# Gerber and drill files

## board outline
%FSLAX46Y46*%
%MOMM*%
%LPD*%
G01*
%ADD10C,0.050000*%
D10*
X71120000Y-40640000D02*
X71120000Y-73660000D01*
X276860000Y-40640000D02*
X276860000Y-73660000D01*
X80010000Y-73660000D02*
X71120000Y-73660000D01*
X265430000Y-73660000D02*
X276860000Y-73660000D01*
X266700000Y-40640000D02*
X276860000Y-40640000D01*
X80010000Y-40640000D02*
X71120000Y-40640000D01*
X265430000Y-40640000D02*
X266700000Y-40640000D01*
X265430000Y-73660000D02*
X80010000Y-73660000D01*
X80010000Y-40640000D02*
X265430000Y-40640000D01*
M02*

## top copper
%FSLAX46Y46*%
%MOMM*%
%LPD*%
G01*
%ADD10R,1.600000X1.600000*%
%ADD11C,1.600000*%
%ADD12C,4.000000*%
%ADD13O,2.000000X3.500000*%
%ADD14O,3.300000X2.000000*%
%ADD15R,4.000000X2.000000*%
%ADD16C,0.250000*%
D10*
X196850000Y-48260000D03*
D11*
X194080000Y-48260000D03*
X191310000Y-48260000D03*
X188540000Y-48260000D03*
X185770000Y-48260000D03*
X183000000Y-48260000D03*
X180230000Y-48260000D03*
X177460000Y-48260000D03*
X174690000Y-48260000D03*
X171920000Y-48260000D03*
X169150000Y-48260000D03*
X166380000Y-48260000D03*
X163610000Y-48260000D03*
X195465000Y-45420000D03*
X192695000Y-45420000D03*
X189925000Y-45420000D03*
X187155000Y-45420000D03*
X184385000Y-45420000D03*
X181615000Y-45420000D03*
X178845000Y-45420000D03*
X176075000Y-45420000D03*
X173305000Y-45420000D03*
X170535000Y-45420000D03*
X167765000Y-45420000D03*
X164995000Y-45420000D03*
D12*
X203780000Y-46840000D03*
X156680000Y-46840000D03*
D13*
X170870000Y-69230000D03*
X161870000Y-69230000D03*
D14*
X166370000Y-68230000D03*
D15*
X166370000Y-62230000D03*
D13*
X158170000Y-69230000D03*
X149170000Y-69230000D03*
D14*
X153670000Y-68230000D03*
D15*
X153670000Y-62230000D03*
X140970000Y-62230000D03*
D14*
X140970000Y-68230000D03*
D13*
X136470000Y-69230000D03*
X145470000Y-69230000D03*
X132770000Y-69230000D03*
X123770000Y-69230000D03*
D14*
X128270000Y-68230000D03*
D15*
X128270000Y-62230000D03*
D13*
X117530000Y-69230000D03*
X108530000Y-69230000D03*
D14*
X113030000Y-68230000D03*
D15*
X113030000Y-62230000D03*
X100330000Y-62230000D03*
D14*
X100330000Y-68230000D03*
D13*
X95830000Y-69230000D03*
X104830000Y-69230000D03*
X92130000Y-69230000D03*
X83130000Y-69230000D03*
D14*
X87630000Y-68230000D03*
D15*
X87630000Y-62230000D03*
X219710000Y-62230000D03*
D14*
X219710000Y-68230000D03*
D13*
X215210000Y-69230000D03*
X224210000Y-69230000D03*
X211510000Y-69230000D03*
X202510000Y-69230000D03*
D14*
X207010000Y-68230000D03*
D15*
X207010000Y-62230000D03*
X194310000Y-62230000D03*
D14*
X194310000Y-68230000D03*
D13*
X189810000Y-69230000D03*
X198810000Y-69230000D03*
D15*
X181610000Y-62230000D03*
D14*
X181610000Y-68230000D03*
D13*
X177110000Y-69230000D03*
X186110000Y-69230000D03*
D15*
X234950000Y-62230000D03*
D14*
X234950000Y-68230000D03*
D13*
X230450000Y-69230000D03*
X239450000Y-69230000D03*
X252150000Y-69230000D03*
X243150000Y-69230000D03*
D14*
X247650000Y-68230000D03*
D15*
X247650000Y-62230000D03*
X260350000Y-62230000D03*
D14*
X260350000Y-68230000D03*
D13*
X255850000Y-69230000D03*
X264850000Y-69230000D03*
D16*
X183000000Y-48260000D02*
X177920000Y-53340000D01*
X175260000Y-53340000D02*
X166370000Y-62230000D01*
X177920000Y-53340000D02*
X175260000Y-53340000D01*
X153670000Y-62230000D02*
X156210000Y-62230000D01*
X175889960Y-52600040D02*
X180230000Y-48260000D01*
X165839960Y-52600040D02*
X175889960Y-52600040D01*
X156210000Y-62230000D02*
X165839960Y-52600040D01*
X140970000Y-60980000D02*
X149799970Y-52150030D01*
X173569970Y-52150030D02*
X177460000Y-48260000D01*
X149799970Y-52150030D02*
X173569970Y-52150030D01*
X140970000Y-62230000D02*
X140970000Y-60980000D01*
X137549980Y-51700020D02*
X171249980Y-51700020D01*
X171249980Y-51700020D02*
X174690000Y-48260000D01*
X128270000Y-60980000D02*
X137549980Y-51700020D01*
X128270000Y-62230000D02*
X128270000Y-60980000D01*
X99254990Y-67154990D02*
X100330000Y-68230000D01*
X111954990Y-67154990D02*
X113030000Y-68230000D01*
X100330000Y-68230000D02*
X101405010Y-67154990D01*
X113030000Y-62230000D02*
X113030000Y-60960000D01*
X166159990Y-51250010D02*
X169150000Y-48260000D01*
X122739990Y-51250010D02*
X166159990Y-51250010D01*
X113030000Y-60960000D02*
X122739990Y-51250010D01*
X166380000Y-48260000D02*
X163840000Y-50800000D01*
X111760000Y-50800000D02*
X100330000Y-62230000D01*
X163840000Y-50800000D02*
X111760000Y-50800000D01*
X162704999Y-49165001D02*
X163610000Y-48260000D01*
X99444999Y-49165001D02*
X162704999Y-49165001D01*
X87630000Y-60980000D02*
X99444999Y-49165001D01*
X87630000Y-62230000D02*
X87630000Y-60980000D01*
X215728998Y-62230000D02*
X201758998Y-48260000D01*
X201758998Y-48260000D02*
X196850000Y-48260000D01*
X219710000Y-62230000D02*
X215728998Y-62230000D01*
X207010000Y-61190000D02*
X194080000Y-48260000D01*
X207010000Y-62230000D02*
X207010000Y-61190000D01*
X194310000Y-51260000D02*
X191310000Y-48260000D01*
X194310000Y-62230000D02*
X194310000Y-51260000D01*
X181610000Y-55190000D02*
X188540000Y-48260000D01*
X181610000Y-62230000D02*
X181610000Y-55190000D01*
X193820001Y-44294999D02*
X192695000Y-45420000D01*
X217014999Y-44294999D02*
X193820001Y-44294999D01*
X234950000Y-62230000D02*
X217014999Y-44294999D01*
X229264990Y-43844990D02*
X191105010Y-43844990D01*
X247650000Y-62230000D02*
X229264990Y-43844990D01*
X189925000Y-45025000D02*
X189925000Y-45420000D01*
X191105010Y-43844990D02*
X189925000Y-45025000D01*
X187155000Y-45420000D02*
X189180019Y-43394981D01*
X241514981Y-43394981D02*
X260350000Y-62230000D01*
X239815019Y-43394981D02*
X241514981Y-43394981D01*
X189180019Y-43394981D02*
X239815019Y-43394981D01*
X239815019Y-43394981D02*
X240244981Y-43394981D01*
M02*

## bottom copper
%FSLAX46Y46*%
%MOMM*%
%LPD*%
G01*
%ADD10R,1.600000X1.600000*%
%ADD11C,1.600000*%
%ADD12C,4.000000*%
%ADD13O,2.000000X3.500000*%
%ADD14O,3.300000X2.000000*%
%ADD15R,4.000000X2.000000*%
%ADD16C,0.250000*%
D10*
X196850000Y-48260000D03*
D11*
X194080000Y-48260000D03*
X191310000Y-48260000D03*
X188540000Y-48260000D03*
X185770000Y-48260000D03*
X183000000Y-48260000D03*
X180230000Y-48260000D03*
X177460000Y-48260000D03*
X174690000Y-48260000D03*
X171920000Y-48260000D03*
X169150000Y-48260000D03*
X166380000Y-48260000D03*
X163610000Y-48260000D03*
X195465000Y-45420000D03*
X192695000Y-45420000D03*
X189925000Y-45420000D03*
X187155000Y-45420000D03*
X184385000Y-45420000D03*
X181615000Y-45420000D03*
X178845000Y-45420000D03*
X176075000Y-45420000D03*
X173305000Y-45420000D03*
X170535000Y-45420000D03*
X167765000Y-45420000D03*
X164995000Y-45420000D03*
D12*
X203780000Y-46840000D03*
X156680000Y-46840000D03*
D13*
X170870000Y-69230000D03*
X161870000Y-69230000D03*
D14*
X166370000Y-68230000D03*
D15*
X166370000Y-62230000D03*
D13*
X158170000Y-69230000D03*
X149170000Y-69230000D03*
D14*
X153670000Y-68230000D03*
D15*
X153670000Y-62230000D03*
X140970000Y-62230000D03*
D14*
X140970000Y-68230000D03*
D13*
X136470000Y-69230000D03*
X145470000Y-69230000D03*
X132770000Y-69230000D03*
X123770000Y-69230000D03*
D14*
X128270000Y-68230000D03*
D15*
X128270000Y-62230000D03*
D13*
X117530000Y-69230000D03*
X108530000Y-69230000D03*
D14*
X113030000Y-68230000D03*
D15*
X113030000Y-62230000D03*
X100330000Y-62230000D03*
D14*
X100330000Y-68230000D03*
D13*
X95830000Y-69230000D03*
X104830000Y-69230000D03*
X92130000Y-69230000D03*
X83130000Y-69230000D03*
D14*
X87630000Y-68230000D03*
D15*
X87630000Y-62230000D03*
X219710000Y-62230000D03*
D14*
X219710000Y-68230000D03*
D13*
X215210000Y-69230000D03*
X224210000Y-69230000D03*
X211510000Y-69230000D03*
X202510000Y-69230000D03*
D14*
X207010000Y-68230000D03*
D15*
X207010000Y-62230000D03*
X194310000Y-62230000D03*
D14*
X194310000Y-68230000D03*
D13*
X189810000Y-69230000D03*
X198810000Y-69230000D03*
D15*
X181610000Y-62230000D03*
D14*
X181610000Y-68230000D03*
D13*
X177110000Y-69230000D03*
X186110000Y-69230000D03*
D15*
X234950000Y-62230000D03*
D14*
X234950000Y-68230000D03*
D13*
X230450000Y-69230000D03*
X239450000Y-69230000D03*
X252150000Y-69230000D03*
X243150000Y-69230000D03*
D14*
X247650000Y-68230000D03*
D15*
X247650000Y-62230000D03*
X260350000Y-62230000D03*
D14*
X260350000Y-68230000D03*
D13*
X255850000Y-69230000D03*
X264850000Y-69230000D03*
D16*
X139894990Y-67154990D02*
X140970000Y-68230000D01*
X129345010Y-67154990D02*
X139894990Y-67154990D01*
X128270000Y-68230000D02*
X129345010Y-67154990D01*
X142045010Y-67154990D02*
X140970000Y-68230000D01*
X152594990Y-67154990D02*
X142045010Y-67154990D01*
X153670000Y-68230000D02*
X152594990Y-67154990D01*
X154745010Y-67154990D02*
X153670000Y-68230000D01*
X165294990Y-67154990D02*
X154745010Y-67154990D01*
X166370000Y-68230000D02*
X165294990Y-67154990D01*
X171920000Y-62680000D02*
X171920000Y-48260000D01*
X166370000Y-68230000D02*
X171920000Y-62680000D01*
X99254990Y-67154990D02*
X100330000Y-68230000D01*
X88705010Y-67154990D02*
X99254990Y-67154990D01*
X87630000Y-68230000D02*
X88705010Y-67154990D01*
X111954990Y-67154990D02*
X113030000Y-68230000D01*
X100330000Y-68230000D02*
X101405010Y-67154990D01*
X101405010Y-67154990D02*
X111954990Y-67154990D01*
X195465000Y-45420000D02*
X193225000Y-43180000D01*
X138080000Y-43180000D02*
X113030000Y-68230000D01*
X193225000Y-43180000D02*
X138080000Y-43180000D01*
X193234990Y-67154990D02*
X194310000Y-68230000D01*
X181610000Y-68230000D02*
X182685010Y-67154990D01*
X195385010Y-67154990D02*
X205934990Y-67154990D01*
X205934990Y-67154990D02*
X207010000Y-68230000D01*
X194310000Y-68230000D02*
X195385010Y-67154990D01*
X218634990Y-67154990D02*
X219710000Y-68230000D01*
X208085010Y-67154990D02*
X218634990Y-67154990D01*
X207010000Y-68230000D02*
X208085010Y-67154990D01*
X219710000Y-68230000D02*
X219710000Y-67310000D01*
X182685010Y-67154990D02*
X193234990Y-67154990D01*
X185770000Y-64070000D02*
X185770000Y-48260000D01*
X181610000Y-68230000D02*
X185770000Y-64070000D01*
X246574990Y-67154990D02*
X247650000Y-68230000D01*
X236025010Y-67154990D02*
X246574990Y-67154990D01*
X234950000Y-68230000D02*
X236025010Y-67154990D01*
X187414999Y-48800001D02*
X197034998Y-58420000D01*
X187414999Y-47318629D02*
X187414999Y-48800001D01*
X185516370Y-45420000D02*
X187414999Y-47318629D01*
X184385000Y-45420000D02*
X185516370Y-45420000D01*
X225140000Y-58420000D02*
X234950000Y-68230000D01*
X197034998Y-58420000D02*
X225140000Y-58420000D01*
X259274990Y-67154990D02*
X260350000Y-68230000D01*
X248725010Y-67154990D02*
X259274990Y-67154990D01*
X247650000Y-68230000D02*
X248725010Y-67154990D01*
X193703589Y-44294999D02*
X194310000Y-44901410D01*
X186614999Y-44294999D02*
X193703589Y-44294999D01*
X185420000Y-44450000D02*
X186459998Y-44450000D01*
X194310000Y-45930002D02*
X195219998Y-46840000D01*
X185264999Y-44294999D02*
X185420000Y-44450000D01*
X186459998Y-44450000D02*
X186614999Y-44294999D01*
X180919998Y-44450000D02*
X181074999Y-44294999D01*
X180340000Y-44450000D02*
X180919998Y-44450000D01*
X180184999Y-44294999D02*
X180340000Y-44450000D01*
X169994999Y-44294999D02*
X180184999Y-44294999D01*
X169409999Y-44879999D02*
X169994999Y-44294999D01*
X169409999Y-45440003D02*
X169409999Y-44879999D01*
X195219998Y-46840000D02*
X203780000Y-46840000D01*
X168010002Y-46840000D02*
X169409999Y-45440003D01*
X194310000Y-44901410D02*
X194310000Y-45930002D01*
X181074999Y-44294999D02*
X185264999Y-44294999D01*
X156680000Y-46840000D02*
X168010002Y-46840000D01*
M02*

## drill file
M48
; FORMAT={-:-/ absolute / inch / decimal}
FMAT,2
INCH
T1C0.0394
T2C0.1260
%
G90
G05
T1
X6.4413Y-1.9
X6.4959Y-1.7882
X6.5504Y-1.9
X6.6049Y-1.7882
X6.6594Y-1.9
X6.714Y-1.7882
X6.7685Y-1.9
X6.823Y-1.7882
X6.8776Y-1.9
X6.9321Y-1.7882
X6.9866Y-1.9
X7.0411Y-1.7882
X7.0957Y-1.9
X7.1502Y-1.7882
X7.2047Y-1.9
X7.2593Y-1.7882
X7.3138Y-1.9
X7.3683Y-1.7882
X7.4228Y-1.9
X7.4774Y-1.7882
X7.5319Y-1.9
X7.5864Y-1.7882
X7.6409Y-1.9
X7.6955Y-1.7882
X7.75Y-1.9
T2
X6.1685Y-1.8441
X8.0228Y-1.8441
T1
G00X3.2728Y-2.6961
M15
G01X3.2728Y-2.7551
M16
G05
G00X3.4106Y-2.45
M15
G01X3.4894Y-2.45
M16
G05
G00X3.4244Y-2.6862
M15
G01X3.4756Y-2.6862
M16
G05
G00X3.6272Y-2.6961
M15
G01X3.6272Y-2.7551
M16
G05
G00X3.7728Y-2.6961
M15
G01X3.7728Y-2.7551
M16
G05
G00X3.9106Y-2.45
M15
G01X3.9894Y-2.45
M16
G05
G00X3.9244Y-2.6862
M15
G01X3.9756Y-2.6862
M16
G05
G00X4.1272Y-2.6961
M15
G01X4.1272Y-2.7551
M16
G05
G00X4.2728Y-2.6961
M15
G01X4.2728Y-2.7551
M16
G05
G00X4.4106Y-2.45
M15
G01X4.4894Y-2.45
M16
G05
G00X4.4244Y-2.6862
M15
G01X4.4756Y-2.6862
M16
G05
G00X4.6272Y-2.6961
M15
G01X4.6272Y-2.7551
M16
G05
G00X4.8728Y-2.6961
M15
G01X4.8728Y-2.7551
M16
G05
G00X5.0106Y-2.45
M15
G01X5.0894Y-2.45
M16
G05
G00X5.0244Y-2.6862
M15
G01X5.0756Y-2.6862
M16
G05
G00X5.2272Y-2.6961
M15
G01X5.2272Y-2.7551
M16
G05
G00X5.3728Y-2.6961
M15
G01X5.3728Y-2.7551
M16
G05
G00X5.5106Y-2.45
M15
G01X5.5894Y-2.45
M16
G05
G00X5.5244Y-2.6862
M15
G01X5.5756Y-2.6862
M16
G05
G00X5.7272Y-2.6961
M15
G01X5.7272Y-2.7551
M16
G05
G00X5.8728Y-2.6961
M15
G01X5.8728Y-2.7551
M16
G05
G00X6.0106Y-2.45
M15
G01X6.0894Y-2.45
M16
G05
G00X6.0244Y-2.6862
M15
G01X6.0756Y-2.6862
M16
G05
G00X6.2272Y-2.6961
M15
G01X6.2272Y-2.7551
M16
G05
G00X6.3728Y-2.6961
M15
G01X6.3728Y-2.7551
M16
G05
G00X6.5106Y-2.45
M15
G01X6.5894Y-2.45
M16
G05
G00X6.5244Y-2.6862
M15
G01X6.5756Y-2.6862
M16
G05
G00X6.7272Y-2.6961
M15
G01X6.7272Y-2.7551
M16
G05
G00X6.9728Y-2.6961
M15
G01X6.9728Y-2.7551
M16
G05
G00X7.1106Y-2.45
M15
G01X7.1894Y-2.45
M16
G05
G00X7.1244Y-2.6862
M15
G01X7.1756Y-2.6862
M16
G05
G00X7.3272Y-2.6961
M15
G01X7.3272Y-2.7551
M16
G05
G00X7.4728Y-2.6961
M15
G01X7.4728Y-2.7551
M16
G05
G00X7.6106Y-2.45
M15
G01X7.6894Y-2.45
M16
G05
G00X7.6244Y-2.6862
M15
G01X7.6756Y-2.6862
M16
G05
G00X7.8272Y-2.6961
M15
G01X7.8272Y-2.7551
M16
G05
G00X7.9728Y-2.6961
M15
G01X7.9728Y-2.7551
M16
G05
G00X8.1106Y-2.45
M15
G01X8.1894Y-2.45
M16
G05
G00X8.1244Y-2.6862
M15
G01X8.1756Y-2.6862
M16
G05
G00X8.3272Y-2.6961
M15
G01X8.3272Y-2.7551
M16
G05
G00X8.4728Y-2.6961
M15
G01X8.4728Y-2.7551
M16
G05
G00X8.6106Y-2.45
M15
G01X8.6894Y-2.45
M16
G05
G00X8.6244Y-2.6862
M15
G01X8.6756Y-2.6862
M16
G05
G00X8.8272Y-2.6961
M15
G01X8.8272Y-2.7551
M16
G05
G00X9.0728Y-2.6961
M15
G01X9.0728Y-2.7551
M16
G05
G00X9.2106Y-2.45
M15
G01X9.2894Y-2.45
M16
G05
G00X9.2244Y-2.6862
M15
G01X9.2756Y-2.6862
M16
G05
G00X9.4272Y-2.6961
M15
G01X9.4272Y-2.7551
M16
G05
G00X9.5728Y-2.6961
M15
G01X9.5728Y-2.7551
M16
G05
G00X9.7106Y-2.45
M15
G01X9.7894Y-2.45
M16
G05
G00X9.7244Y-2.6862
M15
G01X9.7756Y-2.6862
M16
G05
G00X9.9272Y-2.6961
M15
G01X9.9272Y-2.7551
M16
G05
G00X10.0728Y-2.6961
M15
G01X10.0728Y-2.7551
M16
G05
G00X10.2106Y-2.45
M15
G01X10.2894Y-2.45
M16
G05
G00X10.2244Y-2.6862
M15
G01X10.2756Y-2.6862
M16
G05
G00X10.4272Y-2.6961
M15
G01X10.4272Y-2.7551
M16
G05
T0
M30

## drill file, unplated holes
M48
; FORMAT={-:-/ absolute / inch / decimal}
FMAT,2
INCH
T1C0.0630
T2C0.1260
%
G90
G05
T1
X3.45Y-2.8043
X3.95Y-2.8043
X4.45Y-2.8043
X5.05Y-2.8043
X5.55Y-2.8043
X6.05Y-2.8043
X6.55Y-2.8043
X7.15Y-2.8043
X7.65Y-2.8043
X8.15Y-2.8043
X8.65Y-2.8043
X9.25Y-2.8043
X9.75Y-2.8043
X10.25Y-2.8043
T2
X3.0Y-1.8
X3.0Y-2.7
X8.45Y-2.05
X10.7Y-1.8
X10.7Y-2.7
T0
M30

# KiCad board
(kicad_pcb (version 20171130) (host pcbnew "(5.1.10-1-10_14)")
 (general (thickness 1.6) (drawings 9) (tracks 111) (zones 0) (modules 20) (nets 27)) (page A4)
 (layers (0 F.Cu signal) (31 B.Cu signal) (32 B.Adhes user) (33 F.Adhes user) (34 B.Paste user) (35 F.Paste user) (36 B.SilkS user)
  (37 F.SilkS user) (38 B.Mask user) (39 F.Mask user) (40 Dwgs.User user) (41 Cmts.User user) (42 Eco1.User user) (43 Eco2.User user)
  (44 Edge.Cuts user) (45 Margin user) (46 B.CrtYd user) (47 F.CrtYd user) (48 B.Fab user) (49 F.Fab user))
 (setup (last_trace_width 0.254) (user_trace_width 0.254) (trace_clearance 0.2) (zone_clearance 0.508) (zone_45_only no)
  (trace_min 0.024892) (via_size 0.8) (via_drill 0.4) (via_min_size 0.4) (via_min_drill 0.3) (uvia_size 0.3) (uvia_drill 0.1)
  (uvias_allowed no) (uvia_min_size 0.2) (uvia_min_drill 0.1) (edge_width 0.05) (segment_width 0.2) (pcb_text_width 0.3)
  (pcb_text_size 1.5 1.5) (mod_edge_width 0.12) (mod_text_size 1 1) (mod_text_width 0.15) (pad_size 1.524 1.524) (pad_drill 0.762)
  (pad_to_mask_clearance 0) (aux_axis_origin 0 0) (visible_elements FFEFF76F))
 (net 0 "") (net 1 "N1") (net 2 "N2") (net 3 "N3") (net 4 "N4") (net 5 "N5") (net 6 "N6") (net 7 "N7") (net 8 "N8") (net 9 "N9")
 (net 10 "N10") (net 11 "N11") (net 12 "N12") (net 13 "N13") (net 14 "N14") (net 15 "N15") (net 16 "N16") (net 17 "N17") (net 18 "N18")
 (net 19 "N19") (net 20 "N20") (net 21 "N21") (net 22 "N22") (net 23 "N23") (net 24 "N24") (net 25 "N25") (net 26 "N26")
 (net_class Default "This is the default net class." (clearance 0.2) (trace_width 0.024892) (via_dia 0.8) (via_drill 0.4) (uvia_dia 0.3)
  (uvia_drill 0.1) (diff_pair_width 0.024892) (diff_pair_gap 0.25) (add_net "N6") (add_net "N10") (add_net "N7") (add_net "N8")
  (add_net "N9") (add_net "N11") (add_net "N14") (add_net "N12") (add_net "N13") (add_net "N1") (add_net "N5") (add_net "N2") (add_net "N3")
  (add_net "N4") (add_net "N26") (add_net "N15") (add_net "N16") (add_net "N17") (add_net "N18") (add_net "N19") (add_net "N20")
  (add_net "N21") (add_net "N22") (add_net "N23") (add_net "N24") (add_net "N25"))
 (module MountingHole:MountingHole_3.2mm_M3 (layer F.Cu) (at 271.78 45.72)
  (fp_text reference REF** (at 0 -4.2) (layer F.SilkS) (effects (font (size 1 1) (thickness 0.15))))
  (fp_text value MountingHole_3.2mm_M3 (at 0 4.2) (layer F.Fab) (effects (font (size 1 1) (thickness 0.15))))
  (pad 1 np_thru_hole circle (at 0 0) (size 3.2 3.2) (drill 3.2) (layers *.Cu *.Mask)))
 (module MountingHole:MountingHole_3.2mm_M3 (layer F.Cu) (at 271.78 68.58)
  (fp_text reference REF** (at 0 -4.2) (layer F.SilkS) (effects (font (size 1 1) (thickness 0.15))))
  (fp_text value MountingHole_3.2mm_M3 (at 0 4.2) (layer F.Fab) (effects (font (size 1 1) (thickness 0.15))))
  (pad 1 np_thru_hole circle (at 0 0) (size 3.2 3.2) (drill 3.2) (layers *.Cu *.Mask)))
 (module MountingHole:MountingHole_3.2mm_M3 (layer F.Cu) (at 76.2 45.72)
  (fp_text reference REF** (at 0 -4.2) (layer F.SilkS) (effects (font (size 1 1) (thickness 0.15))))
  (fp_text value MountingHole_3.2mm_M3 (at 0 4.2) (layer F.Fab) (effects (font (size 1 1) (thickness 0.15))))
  (pad 1 np_thru_hole circle (at 0 0) (size 3.2 3.2) (drill 3.2) (layers *.Cu *.Mask)))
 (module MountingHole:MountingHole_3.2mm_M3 (layer F.Cu) (at 214.63 52.07)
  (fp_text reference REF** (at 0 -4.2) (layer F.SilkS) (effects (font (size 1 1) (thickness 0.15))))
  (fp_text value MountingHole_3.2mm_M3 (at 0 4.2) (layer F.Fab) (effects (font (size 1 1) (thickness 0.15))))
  (pad 1 np_thru_hole circle (at 0 0) (size 3.2 3.2) (drill 3.2) (layers *.Cu *.Mask)))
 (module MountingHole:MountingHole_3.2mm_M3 (layer F.Cu) (at 76.2 68.58)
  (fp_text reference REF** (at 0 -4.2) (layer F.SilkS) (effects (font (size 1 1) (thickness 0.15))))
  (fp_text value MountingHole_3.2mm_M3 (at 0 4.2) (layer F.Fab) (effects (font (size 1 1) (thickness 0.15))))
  (pad 1 np_thru_hole circle (at 0 0) (size 3.2 3.2) (drill 3.2) (layers *.Cu *.Mask)))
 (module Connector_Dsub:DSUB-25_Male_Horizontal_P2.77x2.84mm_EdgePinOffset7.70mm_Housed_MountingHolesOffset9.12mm (layer F.Cu)
  (at 196.85 48.26 180)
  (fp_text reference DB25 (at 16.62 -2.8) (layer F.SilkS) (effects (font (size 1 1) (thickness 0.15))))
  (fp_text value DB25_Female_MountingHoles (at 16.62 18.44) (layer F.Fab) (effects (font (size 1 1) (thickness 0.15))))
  (pad 1 thru_hole rect (at 0 0 180) (size 1.6 1.6) (drill 1) (layers *.Cu *.Mask) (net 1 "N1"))
  (pad 2 thru_hole circle (at 2.77 0 180) (size 1.6 1.6) (drill 1) (layers *.Cu *.Mask) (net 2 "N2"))
  (pad 3 thru_hole circle (at 5.54 0 180) (size 1.6 1.6) (drill 1) (layers *.Cu *.Mask) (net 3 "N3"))
  (pad 4 thru_hole circle (at 8.31 0 180) (size 1.6 1.6) (drill 1) (layers *.Cu *.Mask) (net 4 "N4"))
  (pad 5 thru_hole circle (at 11.08 0 180) (size 1.6 1.6) (drill 1) (layers *.Cu *.Mask) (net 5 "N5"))
  (pad 6 thru_hole circle (at 13.85 0 180) (size 1.6 1.6) (drill 1) (layers *.Cu *.Mask) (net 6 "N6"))
  (pad 7 thru_hole circle (at 16.62 0 180) (size 1.6 1.6) (drill 1) (layers *.Cu *.Mask) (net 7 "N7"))
  (pad 8 thru_hole circle (at 19.39 0 180) (size 1.6 1.6) (drill 1) (layers *.Cu *.Mask) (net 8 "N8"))
  (pad 9 thru_hole circle (at 22.16 0 180) (size 1.6 1.6) (drill 1) (layers *.Cu *.Mask) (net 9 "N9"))
  (pad 10 thru_hole circle (at 24.93 0 180) (size 1.6 1.6) (drill 1) (layers *.Cu *.Mask) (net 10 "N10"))
  (pad 11 thru_hole circle (at 27.7 0 180) (size 1.6 1.6) (drill 1) (layers *.Cu *.Mask) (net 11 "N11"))
  (pad 12 thru_hole circle (at 30.47 0 180) (size 1.6 1.6) (drill 1) (layers *.Cu *.Mask) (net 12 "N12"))
  (pad 13 thru_hole circle (at 33.24 0 180) (size 1.6 1.6) (drill 1) (layers *.Cu *.Mask) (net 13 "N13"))
  (pad 14 thru_hole circle (at 1.385 2.84 180) (size 1.6 1.6) (drill 1) (layers *.Cu *.Mask) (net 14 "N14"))
  (pad 15 thru_hole circle (at 4.155 2.84 180) (size 1.6 1.6) (drill 1) (layers *.Cu *.Mask) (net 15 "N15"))
  (pad 16 thru_hole circle (at 6.925 2.84 180) (size 1.6 1.6) (drill 1) (layers *.Cu *.Mask) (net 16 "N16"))
  (pad 17 thru_hole circle (at 9.695 2.84 180) (size 1.6 1.6) (drill 1) (layers *.Cu *.Mask) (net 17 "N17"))
  (pad 18 thru_hole circle (at 12.465 2.84 180) (size 1.6 1.6) (drill 1) (layers *.Cu *.Mask) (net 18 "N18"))
  (pad 19 thru_hole circle (at 15.235 2.84 180) (size 1.6 1.6) (drill 1) (layers *.Cu *.Mask) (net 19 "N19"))
  (pad 20 thru_hole circle (at 18.005 2.84 180) (size 1.6 1.6) (drill 1) (layers *.Cu *.Mask) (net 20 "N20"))
  (pad 21 thru_hole circle (at 20.775 2.84 180) (size 1.6 1.6) (drill 1) (layers *.Cu *.Mask) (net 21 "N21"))
  (pad 22 thru_hole circle (at 23.545 2.84 180) (size 1.6 1.6) (drill 1) (layers *.Cu *.Mask) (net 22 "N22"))
  (pad 23 thru_hole circle (at 26.315 2.84 180) (size 1.6 1.6) (drill 1) (layers *.Cu *.Mask) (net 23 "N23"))
  (pad 24 thru_hole circle (at 29.085 2.84 180) (size 1.6 1.6) (drill 1) (layers *.Cu *.Mask) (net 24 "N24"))
  (pad 25 thru_hole circle (at 31.855 2.84 180) (size 1.6 1.6) (drill 1) (layers *.Cu *.Mask) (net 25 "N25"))
  (pad 0 thru_hole circle (at -6.93 1.42 180) (size 4 4) (drill 3.2) (layers *.Cu *.Mask) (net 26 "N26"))
  (pad 0 thru_hole circle (at 40.17 1.42 180) (size 4 4) (drill 3.2) (layers *.Cu *.Mask) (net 26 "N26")))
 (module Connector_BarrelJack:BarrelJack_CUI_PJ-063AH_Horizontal (layer F.Cu) (at 166.37 62.23)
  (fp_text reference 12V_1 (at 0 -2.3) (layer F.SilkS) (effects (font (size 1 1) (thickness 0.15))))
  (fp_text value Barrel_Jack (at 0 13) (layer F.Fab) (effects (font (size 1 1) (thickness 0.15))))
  (pad "" np_thru_hole circle (at 0 9) (size 1.6 1.6) (drill 1.6) (layers *.Cu *.Mask))
  (pad MP thru_hole oval (at 4.5 7) (size 2 3.5) (drill oval 1 2.5) (layers *.Cu *.Mask))
  (pad MP thru_hole oval (at -4.5 7) (size 2 3.5) (drill oval 1 2.5) (layers *.Cu *.Mask))
  (pad 2 thru_hole oval (at 0 6) (size 3.3 2) (drill oval 2.3 1) (layers *.Cu *.Mask) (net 10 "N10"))
  (pad 1 thru_hole rect (at 0 0) (size 4 2) (drill oval 3 1) (layers *.Cu *.Mask) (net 6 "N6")))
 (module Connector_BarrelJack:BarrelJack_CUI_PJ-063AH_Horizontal (layer F.Cu) (at 153.67 62.23)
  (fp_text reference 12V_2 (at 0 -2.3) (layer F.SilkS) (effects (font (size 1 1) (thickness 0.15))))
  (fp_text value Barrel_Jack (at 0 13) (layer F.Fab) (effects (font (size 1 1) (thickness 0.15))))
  (pad "" np_thru_hole circle (at 0 9) (size 1.6 1.6) (drill 1.6) (layers *.Cu *.Mask))
  (pad MP thru_hole oval (at 4.5 7) (size 2 3.5) (drill oval 1 2.5) (layers *.Cu *.Mask))
  (pad MP thru_hole oval (at -4.5 7) (size 2 3.5) (drill oval 1 2.5) (layers *.Cu *.Mask))
  (pad 2 thru_hole oval (at 0 6) (size 3.3 2) (drill oval 2.3 1) (layers *.Cu *.Mask) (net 10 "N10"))
  (pad 1 thru_hole rect (at 0 0) (size 4 2) (drill oval 3 1) (layers *.Cu *.Mask) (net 7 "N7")))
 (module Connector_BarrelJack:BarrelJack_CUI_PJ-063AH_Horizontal (layer F.Cu) (at 140.97 62.23)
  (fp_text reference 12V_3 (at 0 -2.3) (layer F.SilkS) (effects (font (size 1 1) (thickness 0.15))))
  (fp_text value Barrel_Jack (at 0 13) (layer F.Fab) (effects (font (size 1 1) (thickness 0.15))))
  (pad 1 thru_hole rect (at 0 0) (size 4 2) (drill oval 3 1) (layers *.Cu *.Mask) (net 8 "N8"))
  (pad 2 thru_hole oval (at 0 6) (size 3.3 2) (drill oval 2.3 1) (layers *.Cu *.Mask) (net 10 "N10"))
  (pad MP thru_hole oval (at -4.5 7) (size 2 3.5) (drill oval 1 2.5) (layers *.Cu *.Mask))
  (pad MP thru_hole oval (at 4.5 7) (size 2 3.5) (drill oval 1 2.5) (layers *.Cu *.Mask))
  (pad "" np_thru_hole circle (at 0 9) (size 1.6 1.6) (drill 1.6) (layers *.Cu *.Mask)))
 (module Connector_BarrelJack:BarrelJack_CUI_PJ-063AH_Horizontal (layer F.Cu) (at 128.27 62.23)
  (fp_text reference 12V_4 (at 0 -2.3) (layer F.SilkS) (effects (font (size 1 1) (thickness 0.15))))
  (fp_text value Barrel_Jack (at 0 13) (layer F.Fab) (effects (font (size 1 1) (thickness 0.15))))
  (pad "" np_thru_hole circle (at 0 9) (size 1.6 1.6) (drill 1.6) (layers *.Cu *.Mask))
  (pad MP thru_hole oval (at 4.5 7) (size 2 3.5) (drill oval 1 2.5) (layers *.Cu *.Mask))
  (pad MP thru_hole oval (at -4.5 7) (size 2 3.5) (drill oval 1 2.5) (layers *.Cu *.Mask))
  (pad 2 thru_hole oval (at 0 6) (size 3.3 2) (drill oval 2.3 1) (layers *.Cu *.Mask) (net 10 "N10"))
  (pad 1 thru_hole rect (at 0 0) (size 4 2) (drill oval 3 1) (layers *.Cu *.Mask) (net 9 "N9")))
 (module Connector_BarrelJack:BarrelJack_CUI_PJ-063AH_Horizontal (layer F.Cu) (at 113.03 62.23)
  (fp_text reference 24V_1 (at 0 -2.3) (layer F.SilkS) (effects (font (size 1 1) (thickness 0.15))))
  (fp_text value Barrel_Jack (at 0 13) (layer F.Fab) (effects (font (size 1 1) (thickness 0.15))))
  (pad "" np_thru_hole circle (at 0 9) (size 1.6 1.6) (drill 1.6) (layers *.Cu *.Mask))
  (pad MP thru_hole oval (at 4.5 7) (size 2 3.5) (drill oval 1 2.5) (layers *.Cu *.Mask))
  (pad MP thru_hole oval (at -4.5 7) (size 2 3.5) (drill oval 1 2.5) (layers *.Cu *.Mask))
  (pad 2 thru_hole oval (at 0 6) (size 3.3 2) (drill oval 2.3 1) (layers *.Cu *.Mask) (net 14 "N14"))
  (pad 1 thru_hole rect (at 0 0) (size 4 2) (drill oval 3 1) (layers *.Cu *.Mask) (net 11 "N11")))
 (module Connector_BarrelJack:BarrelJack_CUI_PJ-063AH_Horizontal (layer F.Cu) (at 100.33 62.23)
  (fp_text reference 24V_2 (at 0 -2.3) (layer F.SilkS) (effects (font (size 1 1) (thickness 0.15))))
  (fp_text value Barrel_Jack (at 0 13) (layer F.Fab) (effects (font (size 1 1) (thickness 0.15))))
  (pad 1 thru_hole rect (at 0 0) (size 4 2) (drill oval 3 1) (layers *.Cu *.Mask) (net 12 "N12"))
  (pad 2 thru_hole oval (at 0 6) (size 3.3 2) (drill oval 2.3 1) (layers *.Cu *.Mask) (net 14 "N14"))
  (pad MP thru_hole oval (at -4.5 7) (size 2 3.5) (drill oval 1 2.5) (layers *.Cu *.Mask))
  (pad MP thru_hole oval (at 4.5 7) (size 2 3.5) (drill oval 1 2.5) (layers *.Cu *.Mask))
  (pad "" np_thru_hole circle (at 0 9) (size 1.6 1.6) (drill 1.6) (layers *.Cu *.Mask)))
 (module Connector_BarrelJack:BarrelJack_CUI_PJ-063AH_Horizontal (layer F.Cu) (at 87.63 62.23)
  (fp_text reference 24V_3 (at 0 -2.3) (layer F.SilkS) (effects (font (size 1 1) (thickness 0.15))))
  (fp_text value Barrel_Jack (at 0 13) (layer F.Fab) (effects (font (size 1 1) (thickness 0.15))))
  (pad "" np_thru_hole circle (at 0 9) (size 1.6 1.6) (drill 1.6) (layers *.Cu *.Mask))
  (pad MP thru_hole oval (at 4.5 7) (size 2 3.5) (drill oval 1 2.5) (layers *.Cu *.Mask))
  (pad MP thru_hole oval (at -4.5 7) (size 2 3.5) (drill oval 1 2.5) (layers *.Cu *.Mask))
  (pad 2 thru_hole oval (at 0 6) (size 3.3 2) (drill oval 2.3 1) (layers *.Cu *.Mask) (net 14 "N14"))
  (pad 1 thru_hole rect (at 0 0) (size 4 2) (drill oval 3 1) (layers *.Cu *.Mask) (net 13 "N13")))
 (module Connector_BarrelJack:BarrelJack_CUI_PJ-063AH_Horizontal (layer F.Cu) (at 219.71 62.23)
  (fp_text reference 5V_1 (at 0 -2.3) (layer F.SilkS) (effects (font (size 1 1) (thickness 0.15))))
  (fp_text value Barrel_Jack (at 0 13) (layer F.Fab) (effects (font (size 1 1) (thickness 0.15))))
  (pad 1 thru_hole rect (at 0 0) (size 4 2) (drill oval 3 1) (layers *.Cu *.Mask) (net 1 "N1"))
  (pad 2 thru_hole oval (at 0 6) (size 3.3 2) (drill oval 2.3 1) (layers *.Cu *.Mask) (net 5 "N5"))
  (pad MP thru_hole oval (at -4.5 7) (size 2 3.5) (drill oval 1 2.5) (layers *.Cu *.Mask))
  (pad MP thru_hole oval (at 4.5 7) (size 2 3.5) (drill oval 1 2.5) (layers *.Cu *.Mask))
  (pad "" np_thru_hole circle (at 0 9) (size 1.6 1.6) (drill 1.6) (layers *.Cu *.Mask)))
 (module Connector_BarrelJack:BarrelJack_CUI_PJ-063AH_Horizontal (layer F.Cu) (at 207.01 62.23)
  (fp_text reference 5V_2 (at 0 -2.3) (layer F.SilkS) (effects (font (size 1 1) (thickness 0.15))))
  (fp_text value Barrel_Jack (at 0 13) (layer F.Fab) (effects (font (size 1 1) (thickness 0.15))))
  (pad "" np_thru_hole circle (at 0 9) (size 1.6 1.6) (drill 1.6) (layers *.Cu *.Mask))
  (pad MP thru_hole oval (at 4.5 7) (size 2 3.5) (drill oval 1 2.5) (layers *.Cu *.Mask))
  (pad MP thru_hole oval (at -4.5 7) (size 2 3.5) (drill oval 1 2.5) (layers *.Cu *.Mask))
  (pad 2 thru_hole oval (at 0 6) (size 3.3 2) (drill oval 2.3 1) (layers *.Cu *.Mask) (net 5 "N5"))
  (pad 1 thru_hole rect (at 0 0) (size 4 2) (drill oval 3 1) (layers *.Cu *.Mask) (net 2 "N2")))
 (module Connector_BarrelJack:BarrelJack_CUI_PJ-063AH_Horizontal (layer F.Cu) (at 194.31 62.23)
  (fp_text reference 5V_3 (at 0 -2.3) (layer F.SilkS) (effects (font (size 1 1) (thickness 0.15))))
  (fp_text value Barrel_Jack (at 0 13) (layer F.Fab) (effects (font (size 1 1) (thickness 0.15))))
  (pad 1 thru_hole rect (at 0 0) (size 4 2) (drill oval 3 1) (layers *.Cu *.Mask) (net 3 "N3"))
  (pad 2 thru_hole oval (at 0 6) (size 3.3 2) (drill oval 2.3 1) (layers *.Cu *.Mask) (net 5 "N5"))
  (pad MP thru_hole oval (at -4.5 7) (size 2 3.5) (drill oval 1 2.5) (layers *.Cu *.Mask))
  (pad MP thru_hole oval (at 4.5 7) (size 2 3.5) (drill oval 1 2.5) (layers *.Cu *.Mask))
  (pad "" np_thru_hole circle (at 0 9) (size 1.6 1.6) (drill 1.6) (layers *.Cu *.Mask)))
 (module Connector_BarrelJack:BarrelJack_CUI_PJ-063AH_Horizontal (layer F.Cu) (at 181.61 62.23)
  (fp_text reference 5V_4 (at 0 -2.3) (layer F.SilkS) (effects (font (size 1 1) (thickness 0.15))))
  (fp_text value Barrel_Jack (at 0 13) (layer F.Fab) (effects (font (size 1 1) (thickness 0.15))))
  (pad 1 thru_hole rect (at 0 0) (size 4 2) (drill oval 3 1) (layers *.Cu *.Mask) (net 4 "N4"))
  (pad 2 thru_hole oval (at 0 6) (size 3.3 2) (drill oval 2.3 1) (layers *.Cu *.Mask) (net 5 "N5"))
  (pad MP thru_hole oval (at -4.5 7) (size 2 3.5) (drill oval 1 2.5) (layers *.Cu *.Mask))
  (pad MP thru_hole oval (at 4.5 7) (size 2 3.5) (drill oval 1 2.5) (layers *.Cu *.Mask))
  (pad "" np_thru_hole circle (at 0 9) (size 1.6 1.6) (drill 1.6) (layers *.Cu *.Mask)))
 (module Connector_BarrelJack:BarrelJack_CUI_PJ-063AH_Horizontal (layer F.Cu) (at 234.95 62.23)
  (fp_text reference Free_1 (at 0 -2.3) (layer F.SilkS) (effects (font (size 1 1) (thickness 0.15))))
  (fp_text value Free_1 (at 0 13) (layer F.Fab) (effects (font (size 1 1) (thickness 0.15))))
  (pad 1 thru_hole rect (at 0 0) (size 4 2) (drill oval 3 1) (layers *.Cu *.Mask) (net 15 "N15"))
  (pad 2 thru_hole oval (at 0 6) (size 3.3 2) (drill oval 2.3 1) (layers *.Cu *.Mask) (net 18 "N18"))
  (pad MP thru_hole oval (at -4.5 7) (size 2 3.5) (drill oval 1 2.5) (layers *.Cu *.Mask))
  (pad MP thru_hole oval (at 4.5 7) (size 2 3.5) (drill oval 1 2.5) (layers *.Cu *.Mask))
  (pad "" np_thru_hole circle (at 0 9) (size 1.6 1.6) (drill 1.6) (layers *.Cu *.Mask)))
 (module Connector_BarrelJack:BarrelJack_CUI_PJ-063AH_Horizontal (layer F.Cu) (at 247.65 62.23)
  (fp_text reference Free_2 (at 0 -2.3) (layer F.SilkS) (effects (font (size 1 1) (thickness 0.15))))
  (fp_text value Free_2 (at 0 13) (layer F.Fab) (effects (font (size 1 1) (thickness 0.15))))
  (pad "" np_thru_hole circle (at 0 9) (size 1.6 1.6) (drill 1.6) (layers *.Cu *.Mask))
  (pad MP thru_hole oval (at 4.5 7) (size 2 3.5) (drill oval 1 2.5) (layers *.Cu *.Mask))
  (pad MP thru_hole oval (at -4.5 7) (size 2 3.5) (drill oval 1 2.5) (layers *.Cu *.Mask))
  (pad 2 thru_hole oval (at 0 6) (size 3.3 2) (drill oval 2.3 1) (layers *.Cu *.Mask) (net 18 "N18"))
  (pad 1 thru_hole rect (at 0 0) (size 4 2) (drill oval 3 1) (layers *.Cu *.Mask) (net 16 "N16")))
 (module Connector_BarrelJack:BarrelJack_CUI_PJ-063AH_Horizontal (layer F.Cu) (at 260.35 62.23)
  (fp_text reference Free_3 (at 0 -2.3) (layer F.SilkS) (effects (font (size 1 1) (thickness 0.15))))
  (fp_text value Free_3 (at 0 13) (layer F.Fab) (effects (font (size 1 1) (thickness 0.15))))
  (pad 1 thru_hole rect (at 0 0) (size 4 2) (drill oval 3 1) (layers *.Cu *.Mask) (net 17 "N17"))
  (pad 2 thru_hole oval (at 0 6) (size 3.3 2) (drill oval 2.3 1) (layers *.Cu *.Mask) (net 18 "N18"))
  (pad MP thru_hole oval (at -4.5 7) (size 2 3.5) (drill oval 1 2.5) (layers *.Cu *.Mask))
  (pad MP thru_hole oval (at 4.5 7) (size 2 3.5) (drill oval 1 2.5) (layers *.Cu *.Mask))
  (pad "" np_thru_hole circle (at 0 9) (size 1.6 1.6) (drill 1.6) (layers *.Cu *.Mask)))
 (gr_line (start 71.12 40.64) (end 71.12 73.66) (layer Edge.Cuts) (width 0.05))
 (gr_line (start 276.86 40.64) (end 276.86 73.66) (layer Edge.Cuts) (width 0.05))
 (gr_line (start 80.01 73.66) (end 71.12 73.66) (layer Edge.Cuts) (width 0.05))
 (gr_line (start 265.43 73.66) (end 276.86 73.66) (layer Edge.Cuts) (width 0.05))
 (gr_line (start 266.7 40.64) (end 276.86 40.64) (layer Edge.Cuts) (width 0.05))
 (gr_line (start 80.01 40.64) (end 71.12 40.64) (layer Edge.Cuts) (width 0.05))
 (gr_line (start 265.43 40.64) (end 266.7 40.64) (layer Edge.Cuts) (width 0.05))
 (gr_line (start 265.43 73.66) (end 80.01 73.66) (layer Edge.Cuts) (width 0.05))
 (gr_line (start 80.01 40.64) (end 265.43 40.64) (layer Edge.Cuts) (width 0.05))
 (segment (start 139.89499 67.15499) (end 140.97 68.23) (width 0.25) (layer B.Cu) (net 10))
 (segment (start 129.34501 67.15499) (end 139.89499 67.15499) (width 0.25) (layer B.Cu) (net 10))
 (segment (start 128.27 68.23) (end 129.34501 67.15499) (width 0.25) (layer B.Cu) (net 10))
 (segment (start 142.04501 67.15499) (end 140.97 68.23) (width 0.25) (layer B.Cu) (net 10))
 (segment (start 152.59499 67.15499) (end 142.04501 67.15499) (width 0.25) (layer B.Cu) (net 10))
 (segment (start 153.67 68.23) (end 152.59499 67.15499) (width 0.25) (layer B.Cu) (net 10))
 (segment (start 154.74501 67.15499) (end 153.67 68.23) (width 0.25) (layer B.Cu) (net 10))
 (segment (start 165.29499 67.15499) (end 154.74501 67.15499) (width 0.25) (layer B.Cu) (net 10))
 (segment (start 166.37 68.23) (end 165.29499 67.15499) (width 0.25) (layer B.Cu) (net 10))
 (segment (start 171.92 62.68) (end 171.92 48.26) (width 0.25) (layer B.Cu) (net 10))
 (segment (start 166.37 68.23) (end 171.92 62.68) (width 0.25) (layer B.Cu) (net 10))
 (segment (start 183 48.26) (end 177.92 53.34) (width 0.25) (layer F.Cu) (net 6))
 (segment (start 175.26 53.34) (end 166.37 62.23) (width 0.25) (layer F.Cu) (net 6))
 (segment (start 177.92 53.34) (end 175.26 53.34) (width 0.25) (layer F.Cu) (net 6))
 (segment (start 153.67 62.23) (end 156.21 62.23) (width 0.25) (layer F.Cu) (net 7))
 (segment (start 175.88996 52.60004) (end 180.23 48.26) (width 0.25) (layer F.Cu) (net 7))
 (segment (start 165.83996 52.60004) (end 175.88996 52.60004) (width 0.25) (layer F.Cu) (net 7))
 (segment (start 156.21 62.23) (end 165.83996 52.60004) (width 0.25) (layer F.Cu) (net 7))
 (segment (start 140.97 60.98) (end 149.79997 52.15003) (width 0.25) (layer F.Cu) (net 8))
 (segment (start 173.56997 52.15003) (end 177.46 48.26) (width 0.25) (layer F.Cu) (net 8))
 (segment (start 149.79997 52.15003) (end 173.56997 52.15003) (width 0.25) (layer F.Cu) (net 8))
 (segment (start 140.97 62.23) (end 140.97 60.98) (width 0.25) (layer F.Cu) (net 8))
 (segment (start 137.54998 51.70002) (end 171.24998 51.70002) (width 0.25) (layer F.Cu) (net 9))
 (segment (start 171.24998 51.70002) (end 174.69 48.26) (width 0.25) (layer F.Cu) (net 9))
 (segment (start 128.27 60.98) (end 137.54998 51.70002) (width 0.25) (layer F.Cu) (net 9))
 (segment (start 128.27 62.23) (end 128.27 60.98) (width 0.25) (layer F.Cu) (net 9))
 (segment (start 99.25499 67.15499) (end 100.33 68.23) (width 0.25) (layer F.Cu) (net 14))
 (segment (start 111.95499 67.15499) (end 113.03 68.23) (width 0.25) (layer F.Cu) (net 14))
 (segment (start 100.33 68.23) (end 101.40501 67.15499) (width 0.25) (layer F.Cu) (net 14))
 (segment (start 99.25499 67.15499) (end 100.33 68.23) (width 0.25) (layer B.Cu) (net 14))
 (segment (start 88.70501 67.15499) (end 99.25499 67.15499) (width 0.25) (layer B.Cu) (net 14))
 (segment (start 87.63 68.23) (end 88.70501 67.15499) (width 0.25) (layer B.Cu) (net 14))
 (segment (start 111.95499 67.15499) (end 113.03 68.23) (width 0.25) (layer B.Cu) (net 14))
 (segment (start 100.33 68.23) (end 101.40501 67.15499) (width 0.25) (layer B.Cu) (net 14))
 (segment (start 101.40501 67.15499) (end 111.95499 67.15499) (width 0.25) (layer B.Cu) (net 14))
 (segment (start 195.465 45.42) (end 193.225 43.18) (width 0.25) (layer B.Cu) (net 14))
 (segment (start 138.08 43.18) (end 113.03 68.23) (width 0.25) (layer B.Cu) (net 14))
 (segment (start 193.225 43.18) (end 138.08 43.18) (width 0.25) (layer B.Cu) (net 14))
 (segment (start 113.03 62.23) (end 113.03 60.96) (width 0.25) (layer F.Cu) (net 11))
 (segment (start 166.15999 51.25001) (end 169.15 48.26) (width 0.25) (layer F.Cu) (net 11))
 (segment (start 122.73999 51.25001) (end 166.15999 51.25001) (width 0.25) (layer F.Cu) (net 11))
 (segment (start 113.03 60.96) (end 122.73999 51.25001) (width 0.25) (layer F.Cu) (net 11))
 (segment (start 166.38 48.26) (end 163.84 50.8) (width 0.25) (layer F.Cu) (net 12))
 (segment (start 111.76 50.8) (end 100.33 62.23) (width 0.25) (layer F.Cu) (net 12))
 (segment (start 163.84 50.8) (end 111.76 50.8) (width 0.25) (layer F.Cu) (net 12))
 (segment (start 162.704999 49.165001) (end 163.61 48.26) (width 0.25) (layer F.Cu) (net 13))
 (segment (start 99.444999 49.165001) (end 162.704999 49.165001) (width 0.25) (layer F.Cu) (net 13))
 (segment (start 87.63 60.98) (end 99.444999 49.165001) (width 0.25) (layer F.Cu) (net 13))
 (segment (start 87.63 62.23) (end 87.63 60.98) (width 0.25) (layer F.Cu) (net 13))
 (segment (start 215.728998 62.23) (end 201.758998 48.26) (width 0.25) (layer F.Cu) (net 1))
 (segment (start 201.758998 48.26) (end 196.85 48.26) (width 0.25) (layer F.Cu) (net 1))
 (segment (start 219.71 62.23) (end 215.728998 62.23) (width 0.25) (layer F.Cu) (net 1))
 (segment (start 193.23499 67.15499) (end 194.31 68.23) (width 0.25) (layer B.Cu) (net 5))
 (segment (start 181.61 68.23) (end 182.68501 67.15499) (width 0.25) (layer B.Cu) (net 5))
 (segment (start 195.38501 67.15499) (end 205.93499 67.15499) (width 0.25) (layer B.Cu) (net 5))
 (segment (start 205.93499 67.15499) (end 207.01 68.23) (width 0.25) (layer B.Cu) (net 5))
 (segment (start 194.31 68.23) (end 195.38501 67.15499) (width 0.25) (layer B.Cu) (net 5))
 (segment (start 218.63499 67.15499) (end 219.71 68.23) (width 0.25) (layer B.Cu) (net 5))
 (segment (start 208.08501 67.15499) (end 218.63499 67.15499) (width 0.25) (layer B.Cu) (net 5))
 (segment (start 207.01 68.23) (end 208.08501 67.15499) (width 0.25) (layer B.Cu) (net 5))
 (segment (start 219.71 68.23) (end 219.71 67.31) (width 0.25) (layer B.Cu) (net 5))
 (segment (start 182.68501 67.15499) (end 193.23499 67.15499) (width 0.25) (layer B.Cu) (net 5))
 (segment (start 185.77 64.07) (end 185.77 48.26) (width 0.25) (layer B.Cu) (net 5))
 (segment (start 181.61 68.23) (end 185.77 64.07) (width 0.25) (layer B.Cu) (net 5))
 (segment (start 207.01 61.19) (end 194.08 48.26) (width 0.25) (layer F.Cu) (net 2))
 (segment (start 207.01 62.23) (end 207.01 61.19) (width 0.25) (layer F.Cu) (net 2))
 (segment (start 194.31 51.26) (end 191.31 48.26) (width 0.25) (layer F.Cu) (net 3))
 (segment (start 194.31 62.23) (end 194.31 51.26) (width 0.25) (layer F.Cu) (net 3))
 (segment (start 181.61 55.19) (end 188.54 48.26) (width 0.25) (layer F.Cu) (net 4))
 (segment (start 181.61 62.23) (end 181.61 55.19) (width 0.25) (layer F.Cu) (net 4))
 (segment (start 193.820001 44.294999) (end 192.695 45.42) (width 0.25) (layer F.Cu) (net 15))
 (segment (start 217.014999 44.294999) (end 193.820001 44.294999) (width 0.25) (layer F.Cu) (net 15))
 (segment (start 234.95 62.23) (end 217.014999 44.294999) (width 0.25) (layer F.Cu) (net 15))
 (segment (start 229.26499 43.84499) (end 191.10501 43.84499) (width 0.25) (layer F.Cu) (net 16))
 (segment (start 247.65 62.23) (end 229.26499 43.84499) (width 0.25) (layer F.Cu) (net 16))
 (segment (start 189.925 45.025) (end 189.925 45.42) (width 0.25) (layer F.Cu) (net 16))
 (segment (start 191.10501 43.84499) (end 189.925 45.025) (width 0.25) (layer F.Cu) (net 16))
 (segment (start 187.155 45.42) (end 189.180019 43.394981) (width 0.25) (layer F.Cu) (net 17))
 (segment (start 241.514981 43.394981) (end 260.35 62.23) (width 0.25) (layer F.Cu) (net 17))
 (segment (start 239.815019 43.394981) (end 241.514981 43.394981) (width 0.25) (layer F.Cu) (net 17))
 (segment (start 189.180019 43.394981) (end 239.815019 43.394981) (width 0.25) (layer F.Cu) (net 17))
 (segment (start 239.815019 43.394981) (end 240.244981 43.394981) (width 0.25) (layer F.Cu) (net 17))
 (segment (start 246.57499 67.15499) (end 247.65 68.23) (width 0.25) (layer B.Cu) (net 18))
 (segment (start 236.02501 67.15499) (end 246.57499 67.15499) (width 0.25) (layer B.Cu) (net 18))
 (segment (start 234.95 68.23) (end 236.02501 67.15499) (width 0.25) (layer B.Cu) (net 18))
 (segment (start 187.414999 48.800001) (end 197.034998 58.42) (width 0.25) (layer B.Cu) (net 18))
 (segment (start 187.414999 47.318629) (end 187.414999 48.800001) (width 0.25) (layer B.Cu) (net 18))
 (segment (start 185.51637 45.42) (end 187.414999 47.318629) (width 0.25) (layer B.Cu) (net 18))
 (segment (start 184.385 45.42) (end 185.51637 45.42) (width 0.25) (layer B.Cu) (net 18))
 (segment (start 225.14 58.42) (end 234.95 68.23) (width 0.25) (layer B.Cu) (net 18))
 (segment (start 197.034998 58.42) (end 225.14 58.42) (width 0.25) (layer B.Cu) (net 18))
 (segment (start 259.27499 67.15499) (end 260.35 68.23) (width 0.25) (layer B.Cu) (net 18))
 (segment (start 248.72501 67.15499) (end 259.27499 67.15499) (width 0.25) (layer B.Cu) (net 18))
 (segment (start 247.65 68.23) (end 248.72501 67.15499) (width 0.25) (layer B.Cu) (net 18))
 (segment (start 193.703589 44.294999) (end 194.31 44.90141) (width 0.25) (layer B.Cu) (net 26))
 (segment (start 186.614999 44.294999) (end 193.703589 44.294999) (width 0.25) (layer B.Cu) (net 26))
 (segment (start 185.42 44.45) (end 186.459998 44.45) (width 0.25) (layer B.Cu) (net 26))
 (segment (start 194.31 45.930002) (end 195.219998 46.84) (width 0.25) (layer B.Cu) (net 26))
 (segment (start 185.264999 44.294999) (end 185.42 44.45) (width 0.25) (layer B.Cu) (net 26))
 (segment (start 186.459998 44.45) (end 186.614999 44.294999) (width 0.25) (layer B.Cu) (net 26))
 (segment (start 180.919998 44.45) (end 181.074999 44.294999) (width 0.25) (layer B.Cu) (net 26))
 (segment (start 180.34 44.45) (end 180.919998 44.45) (width 0.25) (layer B.Cu) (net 26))
 (segment (start 180.184999 44.294999) (end 180.34 44.45) (width 0.25) (layer B.Cu) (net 26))
 (segment (start 169.994999 44.294999) (end 180.184999 44.294999) (width 0.25) (layer B.Cu) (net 26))
 (segment (start 169.409999 44.879999) (end 169.994999 44.294999) (width 0.25) (layer B.Cu) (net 26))
 (segment (start 169.409999 45.440003) (end 169.409999 44.879999) (width 0.25) (layer B.Cu) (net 26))
 (segment (start 195.219998 46.84) (end 203.78 46.84) (width 0.25) (layer B.Cu) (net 26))
 (segment (start 168.010002 46.84) (end 169.409999 45.440003) (width 0.25) (layer B.Cu) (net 26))
 (segment (start 194.31 44.90141) (end 194.31 45.930002) (width 0.25) (layer B.Cu) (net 26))
 (segment (start 181.074999 44.294999) (end 185.264999 44.294999) (width 0.25) (layer B.Cu) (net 26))
 (segment (start 156.68 46.84) (end 168.010002 46.84) (width 0.25) (layer B.Cu) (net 26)))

